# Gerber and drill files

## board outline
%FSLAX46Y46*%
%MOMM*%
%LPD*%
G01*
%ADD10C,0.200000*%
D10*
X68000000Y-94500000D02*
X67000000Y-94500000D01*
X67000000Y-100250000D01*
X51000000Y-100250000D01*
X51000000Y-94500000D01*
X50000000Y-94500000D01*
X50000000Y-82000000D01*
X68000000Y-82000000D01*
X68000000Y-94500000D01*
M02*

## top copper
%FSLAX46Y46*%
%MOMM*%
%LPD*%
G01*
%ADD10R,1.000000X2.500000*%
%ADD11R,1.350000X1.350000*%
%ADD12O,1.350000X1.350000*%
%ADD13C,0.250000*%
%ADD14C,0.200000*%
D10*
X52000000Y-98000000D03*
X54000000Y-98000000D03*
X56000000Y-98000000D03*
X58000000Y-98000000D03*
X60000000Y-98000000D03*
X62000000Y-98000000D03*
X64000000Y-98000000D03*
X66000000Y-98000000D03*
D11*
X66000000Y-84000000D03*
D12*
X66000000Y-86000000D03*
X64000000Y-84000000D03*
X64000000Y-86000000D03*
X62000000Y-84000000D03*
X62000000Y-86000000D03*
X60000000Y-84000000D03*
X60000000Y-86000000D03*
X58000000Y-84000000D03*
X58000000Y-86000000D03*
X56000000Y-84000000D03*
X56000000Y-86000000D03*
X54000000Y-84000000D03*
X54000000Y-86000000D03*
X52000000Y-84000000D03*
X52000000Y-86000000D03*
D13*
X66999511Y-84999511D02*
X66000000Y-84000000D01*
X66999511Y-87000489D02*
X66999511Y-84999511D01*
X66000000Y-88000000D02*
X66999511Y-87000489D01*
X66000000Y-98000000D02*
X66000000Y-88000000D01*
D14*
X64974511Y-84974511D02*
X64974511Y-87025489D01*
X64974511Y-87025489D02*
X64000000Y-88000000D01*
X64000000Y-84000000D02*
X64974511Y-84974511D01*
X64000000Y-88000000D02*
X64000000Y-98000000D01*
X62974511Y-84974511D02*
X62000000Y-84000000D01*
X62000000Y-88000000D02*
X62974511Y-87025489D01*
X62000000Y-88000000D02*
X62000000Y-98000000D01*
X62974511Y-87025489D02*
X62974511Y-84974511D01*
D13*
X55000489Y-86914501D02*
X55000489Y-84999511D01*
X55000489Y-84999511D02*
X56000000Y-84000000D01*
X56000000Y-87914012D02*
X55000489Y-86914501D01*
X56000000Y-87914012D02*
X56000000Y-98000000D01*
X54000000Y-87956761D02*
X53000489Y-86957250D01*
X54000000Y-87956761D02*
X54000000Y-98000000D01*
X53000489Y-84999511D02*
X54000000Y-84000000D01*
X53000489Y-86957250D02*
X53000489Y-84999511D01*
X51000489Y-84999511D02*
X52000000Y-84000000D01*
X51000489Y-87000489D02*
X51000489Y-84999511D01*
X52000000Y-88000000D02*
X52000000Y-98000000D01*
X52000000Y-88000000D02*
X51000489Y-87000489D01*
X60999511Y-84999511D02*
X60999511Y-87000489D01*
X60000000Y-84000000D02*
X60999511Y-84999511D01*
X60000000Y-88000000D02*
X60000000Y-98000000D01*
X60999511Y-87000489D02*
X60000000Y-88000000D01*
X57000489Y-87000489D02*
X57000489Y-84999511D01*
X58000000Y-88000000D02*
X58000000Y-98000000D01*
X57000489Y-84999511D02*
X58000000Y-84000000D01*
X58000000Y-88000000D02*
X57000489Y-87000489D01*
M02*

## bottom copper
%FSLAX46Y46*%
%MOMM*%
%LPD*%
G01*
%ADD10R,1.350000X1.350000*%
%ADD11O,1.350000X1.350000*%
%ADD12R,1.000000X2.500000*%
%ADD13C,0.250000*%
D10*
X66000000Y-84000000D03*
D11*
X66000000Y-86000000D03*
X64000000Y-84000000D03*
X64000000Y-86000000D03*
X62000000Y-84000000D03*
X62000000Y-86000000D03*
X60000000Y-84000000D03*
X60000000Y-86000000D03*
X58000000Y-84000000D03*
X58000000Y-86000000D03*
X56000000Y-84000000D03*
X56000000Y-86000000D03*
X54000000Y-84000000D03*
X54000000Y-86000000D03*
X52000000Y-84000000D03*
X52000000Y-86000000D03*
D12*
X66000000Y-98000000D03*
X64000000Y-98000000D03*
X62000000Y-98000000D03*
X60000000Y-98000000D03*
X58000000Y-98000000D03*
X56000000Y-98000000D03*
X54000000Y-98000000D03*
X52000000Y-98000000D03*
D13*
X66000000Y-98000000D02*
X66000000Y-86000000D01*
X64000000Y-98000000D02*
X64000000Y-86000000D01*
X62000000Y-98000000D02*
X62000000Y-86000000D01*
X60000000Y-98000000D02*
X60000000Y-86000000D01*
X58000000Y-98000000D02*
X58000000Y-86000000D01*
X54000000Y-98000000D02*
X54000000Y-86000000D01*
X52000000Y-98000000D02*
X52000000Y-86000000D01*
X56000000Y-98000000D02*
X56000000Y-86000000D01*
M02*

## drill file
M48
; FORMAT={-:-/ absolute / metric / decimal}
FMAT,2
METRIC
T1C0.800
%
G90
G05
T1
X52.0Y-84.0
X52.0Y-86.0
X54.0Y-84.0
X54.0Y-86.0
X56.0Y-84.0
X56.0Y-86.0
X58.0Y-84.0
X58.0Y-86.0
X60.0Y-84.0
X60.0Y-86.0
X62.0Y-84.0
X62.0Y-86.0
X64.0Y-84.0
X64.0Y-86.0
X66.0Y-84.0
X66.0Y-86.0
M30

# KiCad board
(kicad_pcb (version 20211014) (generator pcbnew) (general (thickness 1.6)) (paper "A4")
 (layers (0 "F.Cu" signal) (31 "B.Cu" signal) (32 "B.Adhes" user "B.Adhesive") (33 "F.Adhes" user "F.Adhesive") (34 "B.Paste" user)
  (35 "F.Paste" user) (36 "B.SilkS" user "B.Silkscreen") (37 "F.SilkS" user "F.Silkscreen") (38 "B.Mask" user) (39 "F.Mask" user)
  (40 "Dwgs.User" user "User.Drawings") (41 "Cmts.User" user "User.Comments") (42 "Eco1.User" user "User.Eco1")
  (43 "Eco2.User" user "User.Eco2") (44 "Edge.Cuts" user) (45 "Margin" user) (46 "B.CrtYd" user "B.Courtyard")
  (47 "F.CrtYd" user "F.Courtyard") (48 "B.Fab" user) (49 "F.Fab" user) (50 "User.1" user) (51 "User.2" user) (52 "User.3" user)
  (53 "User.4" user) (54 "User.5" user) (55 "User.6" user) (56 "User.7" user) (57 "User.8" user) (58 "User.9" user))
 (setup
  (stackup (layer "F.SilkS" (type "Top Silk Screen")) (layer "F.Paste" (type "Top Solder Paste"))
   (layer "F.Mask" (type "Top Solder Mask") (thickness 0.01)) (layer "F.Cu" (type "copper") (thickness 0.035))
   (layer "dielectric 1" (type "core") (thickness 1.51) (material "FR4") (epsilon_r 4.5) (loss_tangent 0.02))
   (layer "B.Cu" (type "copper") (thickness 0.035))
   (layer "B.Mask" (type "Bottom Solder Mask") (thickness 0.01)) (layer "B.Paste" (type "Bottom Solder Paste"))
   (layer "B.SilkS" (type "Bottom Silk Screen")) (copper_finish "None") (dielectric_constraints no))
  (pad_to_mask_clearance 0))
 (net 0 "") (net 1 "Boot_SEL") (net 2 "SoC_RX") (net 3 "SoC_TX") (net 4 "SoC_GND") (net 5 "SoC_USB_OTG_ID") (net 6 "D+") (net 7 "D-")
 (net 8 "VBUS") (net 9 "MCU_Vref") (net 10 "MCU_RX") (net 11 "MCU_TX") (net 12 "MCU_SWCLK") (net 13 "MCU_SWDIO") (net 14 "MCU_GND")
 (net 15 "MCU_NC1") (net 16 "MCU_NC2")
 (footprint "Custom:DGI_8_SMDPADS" (layer "F.Cu") (at 59 98)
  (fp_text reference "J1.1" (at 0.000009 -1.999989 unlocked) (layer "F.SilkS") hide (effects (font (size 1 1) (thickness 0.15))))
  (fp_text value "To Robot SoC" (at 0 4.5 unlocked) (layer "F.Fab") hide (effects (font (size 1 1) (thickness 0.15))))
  (pad "1" smd rect (at -7 0) (size 1 2.5) (layers "F.Cu" "F.Paste" "F.Mask") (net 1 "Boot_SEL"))
  (pad "2" smd rect (at -5 0) (size 1 2.5) (layers "F.Cu" "F.Paste" "F.Mask") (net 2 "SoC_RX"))
  (pad "3" smd rect (at -3 0) (size 1 2.5) (layers "F.Cu" "F.Paste" "F.Mask") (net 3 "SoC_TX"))
  (pad "4" smd rect (at -1 0) (size 1 2.5) (layers "F.Cu" "F.Paste" "F.Mask") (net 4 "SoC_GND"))
  (pad "5" smd rect (at 1 0) (size 1 2.5) (layers "F.Cu" "F.Paste" "F.Mask") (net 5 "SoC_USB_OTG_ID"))
  (pad "6" smd rect (at 3 0) (size 1 2.5) (layers "F.Cu" "F.Paste" "F.Mask") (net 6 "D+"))
  (pad "7" smd rect (at 5 0) (size 1 2.5) (layers "F.Cu" "F.Paste" "F.Mask") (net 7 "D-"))
  (pad "8" smd rect (at 7 0) (size 1 2.5) (layers "F.Cu" "F.Paste" "F.Mask") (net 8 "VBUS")))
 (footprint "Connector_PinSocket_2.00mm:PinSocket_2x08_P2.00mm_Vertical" (layer "B.Cu") (at 66 84 90)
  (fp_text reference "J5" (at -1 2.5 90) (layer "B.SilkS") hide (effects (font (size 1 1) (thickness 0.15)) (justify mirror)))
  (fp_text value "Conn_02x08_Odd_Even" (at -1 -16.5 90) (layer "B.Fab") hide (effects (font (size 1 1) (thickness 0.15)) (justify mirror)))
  (pad "1" thru_hole rect (at 0 0 90) (size 1.35 1.35) (drill 0.8) (layers *.Cu *.Mask) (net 8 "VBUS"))
  (pad "2" thru_hole oval (at -2 0 90) (size 1.35 1.35) (drill 0.8) (layers *.Cu *.Mask) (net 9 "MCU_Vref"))
  (pad "3" thru_hole oval (at 0 -2 90) (size 1.35 1.35) (drill 0.8) (layers *.Cu *.Mask) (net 7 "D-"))
  (pad "4" thru_hole oval (at -2 -2 90) (size 1.35 1.35) (drill 0.8) (layers *.Cu *.Mask) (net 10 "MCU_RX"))
  (pad "5" thru_hole oval (at 0 -4 90) (size 1.35 1.35) (drill 0.8) (layers *.Cu *.Mask) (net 6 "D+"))
  (pad "6" thru_hole oval (at -2 -4 90) (size 1.35 1.35) (drill 0.8) (layers *.Cu *.Mask) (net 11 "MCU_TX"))
  (pad "7" thru_hole oval (at 0 -6 90) (size 1.35 1.35) (drill 0.8) (layers *.Cu *.Mask) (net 5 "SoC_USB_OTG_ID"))
  (pad "8" thru_hole oval (at -2 -6 90) (size 1.35 1.35) (drill 0.8) (layers *.Cu *.Mask) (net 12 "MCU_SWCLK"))
  (pad "9" thru_hole oval (at 0 -8 90) (size 1.35 1.35) (drill 0.8) (layers *.Cu *.Mask) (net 4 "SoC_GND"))
  (pad "10" thru_hole oval (at -2 -8 90) (size 1.35 1.35) (drill 0.8) (layers *.Cu *.Mask) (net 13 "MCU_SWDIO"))
  (pad "11" thru_hole oval (at 0 -10 90) (size 1.35 1.35) (drill 0.8) (layers *.Cu *.Mask) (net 3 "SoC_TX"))
  (pad "12" thru_hole oval (at -2 -10 90) (size 1.35 1.35) (drill 0.8) (layers *.Cu *.Mask) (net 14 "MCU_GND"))
  (pad "13" thru_hole oval (at 0 -12 90) (size 1.35 1.35) (drill 0.8) (layers *.Cu *.Mask) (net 2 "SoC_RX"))
  (pad "14" thru_hole oval (at -2 -12 90) (size 1.35 1.35) (drill 0.8) (layers *.Cu *.Mask) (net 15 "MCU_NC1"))
  (pad "15" thru_hole oval (at 0 -14 90) (size 1.35 1.35) (drill 0.8) (layers *.Cu *.Mask) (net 1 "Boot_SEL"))
  (pad "16" thru_hole oval (at -2 -14 90) (size 1.35 1.35) (drill 0.8) (layers *.Cu *.Mask) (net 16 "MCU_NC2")))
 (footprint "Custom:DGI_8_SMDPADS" (layer "B.Cu") (at 59 98 180)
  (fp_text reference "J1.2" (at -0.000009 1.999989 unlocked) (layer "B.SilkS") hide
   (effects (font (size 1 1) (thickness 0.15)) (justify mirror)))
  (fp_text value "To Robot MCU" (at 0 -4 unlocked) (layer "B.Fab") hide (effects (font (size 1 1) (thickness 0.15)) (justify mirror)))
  (pad "1" smd rect (at -7 0 180) (size 1 2.5) (layers "B.Cu" "B.Paste" "B.Mask") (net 9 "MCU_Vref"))
  (pad "2" smd rect (at -5 0 180) (size 1 2.5) (layers "B.Cu" "B.Paste" "B.Mask") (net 10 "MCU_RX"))
  (pad "3" smd rect (at -3 0 180) (size 1 2.5) (layers "B.Cu" "B.Paste" "B.Mask") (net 11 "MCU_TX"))
  (pad "4" smd rect (at -1 0 180) (size 1 2.5) (layers "B.Cu" "B.Paste" "B.Mask") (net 12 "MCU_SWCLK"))
  (pad "5" smd rect (at 1 0 180) (size 1 2.5) (layers "B.Cu" "B.Paste" "B.Mask") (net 13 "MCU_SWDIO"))
  (pad "6" smd rect (at 3 0 180) (size 1 2.5) (layers "B.Cu" "B.Paste" "B.Mask") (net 14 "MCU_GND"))
  (pad "7" smd rect (at 5 0 180) (size 1 2.5) (layers "B.Cu" "B.Paste" "B.Mask") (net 15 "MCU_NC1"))
  (pad "8" smd rect (at 7 0 180) (size 1 2.5) (layers "B.Cu" "B.Paste" "B.Mask") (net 16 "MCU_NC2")))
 (gr_poly
  (pts (xy 68 94.5) (xy 67 94.5) (xy 67 100.25) (xy 51 100.25) (xy 51 94.5) (xy 50 94.5) (xy 50 82) (xy 68 82)) (layer "Edge.Cuts")
  (width 0.2) (fill none))
 (segment (start 66 98) (end 66 86) (width 0.25) (layer "B.Cu") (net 9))
 (segment (start 66.999511 84.999511) (end 66 84) (width 0.25) (layer "F.Cu") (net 8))
 (segment (start 66.999511 87.000489) (end 66.999511 84.999511) (width 0.25) (layer "F.Cu") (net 8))
 (segment (start 66 88) (end 66.999511 87.000489) (width 0.25) (layer "F.Cu") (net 8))
 (segment (start 66 98) (end 66 88) (width 0.25) (layer "F.Cu") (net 8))
 (segment (start 64 98) (end 64 86) (width 0.25) (layer "B.Cu") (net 10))
 (segment (start 64.974511 84.974511) (end 64.974511 87.025489) (width 0.2) (layer "F.Cu") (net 7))
 (segment (start 64.974511 87.025489) (end 64 88) (width 0.2) (layer "F.Cu") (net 7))
 (segment (start 64 84) (end 64.974511 84.974511) (width 0.2) (layer "F.Cu") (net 7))
 (segment (start 64 88) (end 64 98) (width 0.2) (layer "F.Cu") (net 7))
 (segment (start 62 98) (end 62 86) (width 0.25) (layer "B.Cu") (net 11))
 (segment (start 62.974511 84.974511) (end 62 84) (width 0.2) (layer "F.Cu") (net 6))
 (segment (start 62 88) (end 62.974511 87.025489) (width 0.2) (layer "F.Cu") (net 6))
 (segment (start 62 88) (end 62 98) (width 0.2) (layer "F.Cu") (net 6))
 (segment (start 62.974511 87.025489) (end 62.974511 84.974511) (width 0.2) (layer "F.Cu") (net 6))
 (segment (start 60 98) (end 60 86) (width 0.25) (layer "B.Cu") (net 12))
 (segment (start 58 98) (end 58 86) (width 0.25) (layer "B.Cu") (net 13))
 (segment (start 55.000489 86.914501) (end 55.000489 84.999511) (width 0.25) (layer "F.Cu") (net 3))
 (segment (start 55.000489 84.999511) (end 56 84) (width 0.25) (layer "F.Cu") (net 3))
 (segment (start 56 87.914012) (end 55.000489 86.914501) (width 0.25) (layer "F.Cu") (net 3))
 (segment (start 56 87.914012) (end 56 98) (width 0.25) (layer "F.Cu") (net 3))
 (segment (start 54 87.956761) (end 53.000489 86.95725) (width 0.25) (layer "F.Cu") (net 2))
 (segment (start 54 87.956761) (end 54 98) (width 0.25) (layer "F.Cu") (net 2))
 (segment (start 53.000489 84.999511) (end 54 84) (width 0.25) (layer "F.Cu") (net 2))
 (segment (start 53.000489 86.95725) (end 53.000489 84.999511) (width 0.25) (layer "F.Cu") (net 2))
 (segment (start 51.000489 84.999511) (end 52 84) (width 0.25) (layer "F.Cu") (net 1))
 (segment (start 51.000489 87.000489) (end 51.000489 84.999511) (width 0.25) (layer "F.Cu") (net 1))
 (segment (start 52 88) (end 52 98) (width 0.25) (layer "F.Cu") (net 1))
 (segment (start 52 88) (end 51.000489 87.000489) (width 0.25) (layer "F.Cu") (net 1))
 (segment (start 60.999511 84.999511) (end 60.999511 87.000489) (width 0.25) (layer "F.Cu") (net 5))
 (segment (start 60 84) (end 60.999511 84.999511) (width 0.25) (layer "F.Cu") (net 5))
 (segment (start 60 88) (end 60 98) (width 0.25) (layer "F.Cu") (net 5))
 (segment (start 60.999511 87.000489) (end 60 88) (width 0.25) (layer "F.Cu") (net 5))
 (segment (start 54 98) (end 54 86) (width 0.25) (layer "B.Cu") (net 15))
 (segment (start 52 98) (end 52 86) (width 0.25) (layer "B.Cu") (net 16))
 (segment (start 57.000489 87.000489) (end 57.000489 84.999511) (width 0.25) (layer "F.Cu") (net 4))
 (segment (start 58 88) (end 58 98) (width 0.25) (layer "F.Cu") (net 4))
 (segment (start 57.000489 84.999511) (end 58 84) (width 0.25) (layer "F.Cu") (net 4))
 (segment (start 58 88) (end 57.000489 87.000489) (width 0.25) (layer "F.Cu") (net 4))
 (segment (start 56 98) (end 56 86) (width 0.25) (layer "B.Cu") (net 14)))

